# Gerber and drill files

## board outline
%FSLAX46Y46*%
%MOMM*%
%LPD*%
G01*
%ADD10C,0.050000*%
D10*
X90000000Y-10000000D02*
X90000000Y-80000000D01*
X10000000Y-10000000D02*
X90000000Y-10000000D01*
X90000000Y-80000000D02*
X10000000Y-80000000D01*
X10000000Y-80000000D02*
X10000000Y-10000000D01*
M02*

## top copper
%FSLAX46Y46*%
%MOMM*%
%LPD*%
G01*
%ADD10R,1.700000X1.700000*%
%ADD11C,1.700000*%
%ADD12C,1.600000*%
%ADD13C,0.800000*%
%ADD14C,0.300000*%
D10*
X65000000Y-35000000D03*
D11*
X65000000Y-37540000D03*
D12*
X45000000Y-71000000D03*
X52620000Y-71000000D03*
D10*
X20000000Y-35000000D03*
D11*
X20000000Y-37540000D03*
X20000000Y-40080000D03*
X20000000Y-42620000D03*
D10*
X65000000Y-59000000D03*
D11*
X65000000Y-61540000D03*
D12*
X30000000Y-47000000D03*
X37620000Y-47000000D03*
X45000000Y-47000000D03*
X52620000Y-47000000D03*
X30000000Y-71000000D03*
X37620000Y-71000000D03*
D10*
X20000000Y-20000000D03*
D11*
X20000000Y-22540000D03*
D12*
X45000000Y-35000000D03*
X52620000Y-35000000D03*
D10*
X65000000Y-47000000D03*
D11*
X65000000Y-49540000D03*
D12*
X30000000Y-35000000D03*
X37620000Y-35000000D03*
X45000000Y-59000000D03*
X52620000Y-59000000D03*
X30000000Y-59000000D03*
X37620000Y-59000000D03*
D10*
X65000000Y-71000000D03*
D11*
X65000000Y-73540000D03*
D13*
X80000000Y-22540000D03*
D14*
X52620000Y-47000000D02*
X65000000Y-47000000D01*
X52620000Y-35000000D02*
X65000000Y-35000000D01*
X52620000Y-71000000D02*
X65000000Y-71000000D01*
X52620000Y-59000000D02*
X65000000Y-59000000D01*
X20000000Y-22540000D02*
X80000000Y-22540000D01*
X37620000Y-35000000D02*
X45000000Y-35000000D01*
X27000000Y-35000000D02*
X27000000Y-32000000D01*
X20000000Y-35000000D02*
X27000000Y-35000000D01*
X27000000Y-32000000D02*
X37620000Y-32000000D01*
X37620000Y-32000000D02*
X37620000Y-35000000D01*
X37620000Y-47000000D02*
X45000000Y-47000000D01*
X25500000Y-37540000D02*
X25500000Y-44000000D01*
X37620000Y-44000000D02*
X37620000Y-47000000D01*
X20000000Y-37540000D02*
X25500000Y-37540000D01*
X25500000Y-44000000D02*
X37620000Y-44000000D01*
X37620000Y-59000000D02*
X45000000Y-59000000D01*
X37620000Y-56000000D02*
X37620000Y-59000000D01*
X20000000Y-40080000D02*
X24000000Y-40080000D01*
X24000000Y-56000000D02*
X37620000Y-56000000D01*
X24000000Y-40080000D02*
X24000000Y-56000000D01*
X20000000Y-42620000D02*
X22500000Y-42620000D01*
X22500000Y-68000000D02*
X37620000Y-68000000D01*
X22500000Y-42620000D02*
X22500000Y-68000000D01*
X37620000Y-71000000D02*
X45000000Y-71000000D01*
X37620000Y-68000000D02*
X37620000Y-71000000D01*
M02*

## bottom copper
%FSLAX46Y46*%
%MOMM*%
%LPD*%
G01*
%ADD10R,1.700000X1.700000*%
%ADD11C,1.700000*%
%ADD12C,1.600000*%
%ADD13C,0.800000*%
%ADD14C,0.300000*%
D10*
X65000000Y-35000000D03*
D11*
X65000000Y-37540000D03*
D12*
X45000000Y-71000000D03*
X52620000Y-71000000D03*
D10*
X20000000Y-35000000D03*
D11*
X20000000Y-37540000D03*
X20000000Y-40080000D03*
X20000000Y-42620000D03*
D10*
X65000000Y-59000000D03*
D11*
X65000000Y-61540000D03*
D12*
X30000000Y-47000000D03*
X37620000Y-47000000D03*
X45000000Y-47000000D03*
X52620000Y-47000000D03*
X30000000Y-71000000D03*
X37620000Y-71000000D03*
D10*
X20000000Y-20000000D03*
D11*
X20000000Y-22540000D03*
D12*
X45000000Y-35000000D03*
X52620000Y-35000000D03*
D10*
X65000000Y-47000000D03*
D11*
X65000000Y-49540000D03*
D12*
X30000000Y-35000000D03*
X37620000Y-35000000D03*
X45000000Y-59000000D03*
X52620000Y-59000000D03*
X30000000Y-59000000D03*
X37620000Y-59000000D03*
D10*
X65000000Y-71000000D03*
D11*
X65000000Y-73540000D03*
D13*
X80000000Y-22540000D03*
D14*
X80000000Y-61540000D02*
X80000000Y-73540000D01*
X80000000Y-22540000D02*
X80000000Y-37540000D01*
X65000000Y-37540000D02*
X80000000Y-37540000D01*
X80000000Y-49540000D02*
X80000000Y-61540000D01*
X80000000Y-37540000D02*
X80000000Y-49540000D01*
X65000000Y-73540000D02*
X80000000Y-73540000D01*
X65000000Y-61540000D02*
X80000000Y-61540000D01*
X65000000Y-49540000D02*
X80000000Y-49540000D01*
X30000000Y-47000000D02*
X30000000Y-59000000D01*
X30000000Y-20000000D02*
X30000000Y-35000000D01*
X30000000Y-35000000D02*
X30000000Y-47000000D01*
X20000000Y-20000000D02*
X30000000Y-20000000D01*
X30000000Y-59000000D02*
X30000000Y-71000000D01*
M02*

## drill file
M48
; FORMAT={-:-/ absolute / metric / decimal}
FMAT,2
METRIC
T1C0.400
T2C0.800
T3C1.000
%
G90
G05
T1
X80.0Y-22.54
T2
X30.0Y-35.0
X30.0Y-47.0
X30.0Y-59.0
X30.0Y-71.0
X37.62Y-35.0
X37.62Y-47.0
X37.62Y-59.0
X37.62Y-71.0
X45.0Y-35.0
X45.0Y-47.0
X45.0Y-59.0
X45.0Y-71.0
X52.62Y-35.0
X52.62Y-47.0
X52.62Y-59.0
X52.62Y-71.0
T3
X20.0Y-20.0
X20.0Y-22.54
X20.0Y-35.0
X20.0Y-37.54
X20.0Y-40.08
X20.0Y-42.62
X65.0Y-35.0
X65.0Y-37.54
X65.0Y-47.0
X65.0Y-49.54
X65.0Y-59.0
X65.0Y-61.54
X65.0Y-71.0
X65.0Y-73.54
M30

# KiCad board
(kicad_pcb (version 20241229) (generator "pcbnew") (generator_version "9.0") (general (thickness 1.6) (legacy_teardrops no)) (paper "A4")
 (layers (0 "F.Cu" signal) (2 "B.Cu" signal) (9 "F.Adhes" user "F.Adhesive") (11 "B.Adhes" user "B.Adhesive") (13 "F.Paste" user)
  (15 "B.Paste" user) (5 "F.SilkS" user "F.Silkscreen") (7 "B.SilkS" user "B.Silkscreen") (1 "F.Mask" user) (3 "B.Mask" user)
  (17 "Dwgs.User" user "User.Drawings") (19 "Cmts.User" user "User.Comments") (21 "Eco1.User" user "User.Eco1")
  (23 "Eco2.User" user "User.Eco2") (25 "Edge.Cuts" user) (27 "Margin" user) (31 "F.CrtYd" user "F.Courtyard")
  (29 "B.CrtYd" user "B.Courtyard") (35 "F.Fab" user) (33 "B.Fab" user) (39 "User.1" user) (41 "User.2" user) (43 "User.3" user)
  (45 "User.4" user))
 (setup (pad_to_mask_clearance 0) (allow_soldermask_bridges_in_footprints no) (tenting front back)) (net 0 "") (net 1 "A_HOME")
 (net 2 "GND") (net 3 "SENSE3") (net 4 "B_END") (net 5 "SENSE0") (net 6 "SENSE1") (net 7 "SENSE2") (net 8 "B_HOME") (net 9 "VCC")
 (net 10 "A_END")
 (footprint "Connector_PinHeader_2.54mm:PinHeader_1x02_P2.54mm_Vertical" (layer "F.Cu") (at 65 35)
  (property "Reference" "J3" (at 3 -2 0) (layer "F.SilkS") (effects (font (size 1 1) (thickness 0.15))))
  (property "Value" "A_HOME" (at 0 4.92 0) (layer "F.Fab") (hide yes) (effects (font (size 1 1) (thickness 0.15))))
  (pad "1" thru_hole rect (at 0 0) (size 1.7 1.7) (drill 1) (layers "*.Cu" "*.Mask") (remove_unused_layers no) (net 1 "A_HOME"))
  (pad "2" thru_hole circle (at 0 2.54) (size 1.7 1.7) (drill 1) (layers "*.Cu" "*.Mask") (remove_unused_layers no) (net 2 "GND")))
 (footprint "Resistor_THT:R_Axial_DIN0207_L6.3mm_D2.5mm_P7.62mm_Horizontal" (layer "F.Cu") (at 45 71)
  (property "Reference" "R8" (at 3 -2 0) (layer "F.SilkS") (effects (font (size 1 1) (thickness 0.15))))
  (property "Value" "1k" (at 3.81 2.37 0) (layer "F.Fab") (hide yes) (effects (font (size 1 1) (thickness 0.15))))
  (pad "1" thru_hole circle (at 0 0) (size 1.6 1.6) (drill 0.8) (layers "*.Cu" "*.Mask") (remove_unused_layers no) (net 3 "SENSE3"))
  (pad "2" thru_hole circle (at 7.62 0) (size 1.6 1.6) (drill 0.8) (layers "*.Cu" "*.Mask") (remove_unused_layers no) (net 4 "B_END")))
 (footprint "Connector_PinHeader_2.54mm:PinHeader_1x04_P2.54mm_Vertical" (layer "F.Cu") (at 20 35)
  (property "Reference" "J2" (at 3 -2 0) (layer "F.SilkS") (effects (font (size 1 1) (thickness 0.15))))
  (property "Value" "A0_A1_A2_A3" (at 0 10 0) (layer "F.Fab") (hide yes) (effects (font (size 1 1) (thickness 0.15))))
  (pad "1" thru_hole rect (at 0 0) (size 1.7 1.7) (drill 1) (layers "*.Cu" "*.Mask") (remove_unused_layers no) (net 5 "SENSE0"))
  (pad "2" thru_hole circle (at 0 2.54) (size 1.7 1.7) (drill 1) (layers "*.Cu" "*.Mask") (remove_unused_layers no) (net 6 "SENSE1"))
  (pad "3" thru_hole circle (at 0 5.08) (size 1.7 1.7) (drill 1) (layers "*.Cu" "*.Mask") (remove_unused_layers no) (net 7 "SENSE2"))
  (pad "4" thru_hole circle (at 0 7.62) (size 1.7 1.7) (drill 1) (layers "*.Cu" "*.Mask") (remove_unused_layers no) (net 3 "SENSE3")))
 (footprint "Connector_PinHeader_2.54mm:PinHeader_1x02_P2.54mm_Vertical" (layer "F.Cu") (at 65 59)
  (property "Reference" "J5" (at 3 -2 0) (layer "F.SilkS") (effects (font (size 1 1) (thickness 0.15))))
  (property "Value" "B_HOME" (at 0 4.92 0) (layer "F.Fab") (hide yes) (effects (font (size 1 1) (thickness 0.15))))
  (pad "1" thru_hole rect (at 0 0) (size 1.7 1.7) (drill 1) (layers "*.Cu" "*.Mask") (remove_unused_layers no) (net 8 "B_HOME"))
  (pad "2" thru_hole circle (at 0 2.54) (size 1.7 1.7) (drill 1) (layers "*.Cu" "*.Mask") (remove_unused_layers no) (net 2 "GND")))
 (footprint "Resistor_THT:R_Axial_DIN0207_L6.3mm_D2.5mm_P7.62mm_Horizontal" (layer "F.Cu") (at 30 47)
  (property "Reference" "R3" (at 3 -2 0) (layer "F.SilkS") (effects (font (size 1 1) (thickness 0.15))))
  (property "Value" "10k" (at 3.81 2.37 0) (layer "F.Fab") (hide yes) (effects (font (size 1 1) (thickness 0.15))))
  (pad "1" thru_hole circle (at 0 0) (size 1.6 1.6) (drill 0.8) (layers "*.Cu" "*.Mask") (remove_unused_layers no) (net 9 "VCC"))
  (pad "2" thru_hole circle (at 7.62 0) (size 1.6 1.6) (drill 0.8) (layers "*.Cu" "*.Mask") (remove_unused_layers no) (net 6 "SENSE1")))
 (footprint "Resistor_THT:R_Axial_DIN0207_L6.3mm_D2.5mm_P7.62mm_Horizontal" (layer "F.Cu") (at 45 47)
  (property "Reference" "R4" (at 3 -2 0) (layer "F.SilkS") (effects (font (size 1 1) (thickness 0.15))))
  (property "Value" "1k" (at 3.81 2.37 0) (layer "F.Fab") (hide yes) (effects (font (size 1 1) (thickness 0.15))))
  (pad "1" thru_hole circle (at 0 0) (size 1.6 1.6) (drill 0.8) (layers "*.Cu" "*.Mask") (remove_unused_layers no) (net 6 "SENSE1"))
  (pad "2" thru_hole circle (at 7.62 0) (size 1.6 1.6) (drill 0.8) (layers "*.Cu" "*.Mask") (remove_unused_layers no) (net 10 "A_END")))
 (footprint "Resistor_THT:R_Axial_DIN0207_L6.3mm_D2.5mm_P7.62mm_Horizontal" (layer "F.Cu") (at 30 71)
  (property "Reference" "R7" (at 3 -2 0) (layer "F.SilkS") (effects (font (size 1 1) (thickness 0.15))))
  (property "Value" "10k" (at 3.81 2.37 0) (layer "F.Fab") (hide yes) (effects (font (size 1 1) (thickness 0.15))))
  (pad "1" thru_hole circle (at 0 0) (size 1.6 1.6) (drill 0.8) (layers "*.Cu" "*.Mask") (remove_unused_layers no) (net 9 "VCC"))
  (pad "2" thru_hole circle (at 7.62 0) (size 1.6 1.6) (drill 0.8) (layers "*.Cu" "*.Mask") (remove_unused_layers no) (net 3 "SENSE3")))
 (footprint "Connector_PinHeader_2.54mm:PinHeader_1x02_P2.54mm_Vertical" (layer "F.Cu") (at 20 20)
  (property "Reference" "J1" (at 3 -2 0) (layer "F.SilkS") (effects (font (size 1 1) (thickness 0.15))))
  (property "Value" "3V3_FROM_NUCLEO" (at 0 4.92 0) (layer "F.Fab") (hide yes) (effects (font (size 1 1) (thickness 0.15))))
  (pad "1" thru_hole rect (at 0 0) (size 1.7 1.7) (drill 1) (layers "*.Cu" "*.Mask") (remove_unused_layers no) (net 9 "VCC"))
  (pad "2" thru_hole circle (at 0 2.54) (size 1.7 1.7) (drill 1) (layers "*.Cu" "*.Mask") (remove_unused_layers no) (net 2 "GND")))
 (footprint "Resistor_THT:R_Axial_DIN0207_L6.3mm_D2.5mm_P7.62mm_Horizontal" (layer "F.Cu") (at 45 35)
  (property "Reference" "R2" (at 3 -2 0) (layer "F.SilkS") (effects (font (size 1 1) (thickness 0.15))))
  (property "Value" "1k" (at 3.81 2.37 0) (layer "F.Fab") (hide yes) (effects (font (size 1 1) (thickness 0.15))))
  (pad "1" thru_hole circle (at 0 0) (size 1.6 1.6) (drill 0.8) (layers "*.Cu" "*.Mask") (remove_unused_layers no) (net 5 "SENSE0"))
  (pad "2" thru_hole circle (at 7.62 0) (size 1.6 1.6) (drill 0.8) (layers "*.Cu" "*.Mask") (remove_unused_layers no) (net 1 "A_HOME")))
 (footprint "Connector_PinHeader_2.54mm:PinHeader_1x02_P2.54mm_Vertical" (layer "F.Cu") (at 65 47)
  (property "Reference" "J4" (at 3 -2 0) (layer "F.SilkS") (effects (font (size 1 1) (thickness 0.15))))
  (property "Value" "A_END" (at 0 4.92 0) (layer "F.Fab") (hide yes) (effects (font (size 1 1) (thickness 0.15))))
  (pad "1" thru_hole rect (at 0 0) (size 1.7 1.7) (drill 1) (layers "*.Cu" "*.Mask") (remove_unused_layers no) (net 10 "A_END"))
  (pad "2" thru_hole circle (at 0 2.54) (size 1.7 1.7) (drill 1) (layers "*.Cu" "*.Mask") (remove_unused_layers no) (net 2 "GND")))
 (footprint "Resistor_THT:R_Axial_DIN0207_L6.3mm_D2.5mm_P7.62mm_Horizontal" (layer "F.Cu") (at 30 35)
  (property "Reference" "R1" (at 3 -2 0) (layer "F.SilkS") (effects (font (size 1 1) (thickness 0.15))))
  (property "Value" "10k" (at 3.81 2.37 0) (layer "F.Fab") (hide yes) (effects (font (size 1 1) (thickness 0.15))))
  (pad "1" thru_hole circle (at 0 0) (size 1.6 1.6) (drill 0.8) (layers "*.Cu" "*.Mask") (remove_unused_layers no) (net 9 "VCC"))
  (pad "2" thru_hole circle (at 7.62 0) (size 1.6 1.6) (drill 0.8) (layers "*.Cu" "*.Mask") (remove_unused_layers no) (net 5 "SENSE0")))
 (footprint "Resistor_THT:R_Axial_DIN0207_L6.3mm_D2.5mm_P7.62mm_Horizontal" (layer "F.Cu") (at 45 59)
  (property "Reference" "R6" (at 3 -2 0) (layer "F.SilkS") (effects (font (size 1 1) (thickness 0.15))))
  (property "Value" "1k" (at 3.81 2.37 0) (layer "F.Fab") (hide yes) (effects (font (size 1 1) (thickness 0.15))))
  (pad "1" thru_hole circle (at 0 0) (size 1.6 1.6) (drill 0.8) (layers "*.Cu" "*.Mask") (remove_unused_layers no) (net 7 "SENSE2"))
  (pad "2" thru_hole circle (at 7.62 0) (size 1.6 1.6) (drill 0.8) (layers "*.Cu" "*.Mask") (remove_unused_layers no) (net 8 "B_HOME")))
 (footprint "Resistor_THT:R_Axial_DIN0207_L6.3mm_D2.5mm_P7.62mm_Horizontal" (layer "F.Cu") (at 30 59)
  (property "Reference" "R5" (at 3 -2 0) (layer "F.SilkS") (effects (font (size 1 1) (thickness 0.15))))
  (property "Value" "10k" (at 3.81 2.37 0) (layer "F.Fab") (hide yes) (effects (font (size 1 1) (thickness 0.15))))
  (pad "1" thru_hole circle (at 0 0) (size 1.6 1.6) (drill 0.8) (layers "*.Cu" "*.Mask") (remove_unused_layers no) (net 9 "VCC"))
  (pad "2" thru_hole circle (at 7.62 0) (size 1.6 1.6) (drill 0.8) (layers "*.Cu" "*.Mask") (remove_unused_layers no) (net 7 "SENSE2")))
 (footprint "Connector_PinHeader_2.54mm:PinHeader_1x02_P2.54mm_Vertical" (layer "F.Cu") (at 65 71)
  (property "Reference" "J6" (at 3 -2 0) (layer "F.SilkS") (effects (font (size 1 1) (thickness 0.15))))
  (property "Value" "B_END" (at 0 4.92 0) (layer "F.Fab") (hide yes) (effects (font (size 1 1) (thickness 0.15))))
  (pad "1" thru_hole rect (at 0 0) (size 1.7 1.7) (drill 1) (layers "*.Cu" "*.Mask") (remove_unused_layers no) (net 4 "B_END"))
  (pad "2" thru_hole circle (at 0 2.54) (size 1.7 1.7) (drill 1) (layers "*.Cu" "*.Mask") (remove_unused_layers no) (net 2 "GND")))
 (gr_line (start 90 10) (end 90 80) (stroke (width 0.05) (type default)) (layer "Edge.Cuts"))
 (gr_line (start 10 10) (end 90 10) (stroke (width 0.05) (type default)) (layer "Edge.Cuts"))
 (gr_line (start 90 80) (end 10 80) (stroke (width 0.05) (type default)) (layer "Edge.Cuts"))
 (gr_line (start 10 80) (end 10 10) (stroke (width 0.05) (type default)) (layer "Edge.Cuts"))
 (segment (start 52.62 47) (end 65 47) (width 0.3) (layer "F.Cu") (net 10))
 (segment (start 52.62 35) (end 65 35) (width 0.3) (layer "F.Cu") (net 1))
 (segment (start 52.62 71) (end 65 71) (width 0.3) (layer "F.Cu") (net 4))
 (segment (start 52.62 59) (end 65 59) (width 0.3) (layer "F.Cu") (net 8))
 (segment (start 20 22.54) (end 80 22.54) (width 0.3) (layer "F.Cu") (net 2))
 (via (at 80 22.54) (size 0.8) (drill 0.4) (layers "F.Cu" "B.Cu") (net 2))
 (segment (start 80 61.54) (end 80 73.54) (width 0.3) (layer "B.Cu") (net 2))
 (segment (start 80 22.54) (end 80 37.54) (width 0.3) (layer "B.Cu") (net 2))
 (segment (start 65 37.54) (end 80 37.54) (width 0.3) (layer "B.Cu") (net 2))
 (segment (start 80 49.54) (end 80 61.54) (width 0.3) (layer "B.Cu") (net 2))
 (segment (start 80 37.54) (end 80 49.54) (width 0.3) (layer "B.Cu") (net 2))
 (segment (start 65 73.54) (end 80 73.54) (width 0.3) (layer "B.Cu") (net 2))
 (segment (start 65 61.54) (end 80 61.54) (width 0.3) (layer "B.Cu") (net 2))
 (segment (start 65 49.54) (end 80 49.54) (width 0.3) (layer "B.Cu") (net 2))
 (segment (start 37.62 35) (end 45 35) (width 0.3) (layer "F.Cu") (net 5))
 (segment (start 27 35) (end 27 32) (width 0.3) (layer "F.Cu") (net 5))
 (segment (start 20 35) (end 27 35) (width 0.3) (layer "F.Cu") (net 5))
 (segment (start 27 32) (end 37.62 32) (width 0.3) (layer "F.Cu") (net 5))
 (segment (start 37.62 32) (end 37.62 35) (width 0.3) (layer "F.Cu") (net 5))
 (segment (start 37.62 47) (end 45 47) (width 0.3) (layer "F.Cu") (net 6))
 (segment (start 25.5 37.54) (end 25.5 44) (width 0.3) (layer "F.Cu") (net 6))
 (segment (start 37.62 44) (end 37.62 47) (width 0.3) (layer "F.Cu") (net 6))
 (segment (start 20 37.54) (end 25.5 37.54) (width 0.3) (layer "F.Cu") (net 6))
 (segment (start 25.5 44) (end 37.62 44) (width 0.3) (layer "F.Cu") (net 6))
 (segment (start 37.62 59) (end 45 59) (width 0.3) (layer "F.Cu") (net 7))
 (segment (start 37.62 56) (end 37.62 59) (width 0.3) (layer "F.Cu") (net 7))
 (segment (start 20 40.08) (end 24 40.08) (width 0.3) (layer "F.Cu") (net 7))
 (segment (start 24 56) (end 37.62 56) (width 0.3) (layer "F.Cu") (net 7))
 (segment (start 24 40.08) (end 24 56) (width 0.3) (layer "F.Cu") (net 7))
 (segment (start 20 42.62) (end 22.5 42.62) (width 0.3) (layer "F.Cu") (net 3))
 (segment (start 22.5 68) (end 37.62 68) (width 0.3) (layer "F.Cu") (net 3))
 (segment (start 22.5 42.62) (end 22.5 68) (width 0.3) (layer "F.Cu") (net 3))
 (segment (start 37.62 71) (end 45 71) (width 0.3) (layer "F.Cu") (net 3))
 (segment (start 37.62 68) (end 37.62 71) (width 0.3) (layer "F.Cu") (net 3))
 (segment (start 30 47) (end 30 59) (width 0.3) (layer "B.Cu") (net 9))
 (segment (start 30 20) (end 30 35) (width 0.3) (layer "B.Cu") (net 9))
 (segment (start 30 35) (end 30 47) (width 0.3) (layer "B.Cu") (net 9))
 (segment (start 20 20) (end 30 20) (width 0.3) (layer "B.Cu") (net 9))
 (segment (start 30 59) (end 30 71) (width 0.3) (layer "B.Cu") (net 9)))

